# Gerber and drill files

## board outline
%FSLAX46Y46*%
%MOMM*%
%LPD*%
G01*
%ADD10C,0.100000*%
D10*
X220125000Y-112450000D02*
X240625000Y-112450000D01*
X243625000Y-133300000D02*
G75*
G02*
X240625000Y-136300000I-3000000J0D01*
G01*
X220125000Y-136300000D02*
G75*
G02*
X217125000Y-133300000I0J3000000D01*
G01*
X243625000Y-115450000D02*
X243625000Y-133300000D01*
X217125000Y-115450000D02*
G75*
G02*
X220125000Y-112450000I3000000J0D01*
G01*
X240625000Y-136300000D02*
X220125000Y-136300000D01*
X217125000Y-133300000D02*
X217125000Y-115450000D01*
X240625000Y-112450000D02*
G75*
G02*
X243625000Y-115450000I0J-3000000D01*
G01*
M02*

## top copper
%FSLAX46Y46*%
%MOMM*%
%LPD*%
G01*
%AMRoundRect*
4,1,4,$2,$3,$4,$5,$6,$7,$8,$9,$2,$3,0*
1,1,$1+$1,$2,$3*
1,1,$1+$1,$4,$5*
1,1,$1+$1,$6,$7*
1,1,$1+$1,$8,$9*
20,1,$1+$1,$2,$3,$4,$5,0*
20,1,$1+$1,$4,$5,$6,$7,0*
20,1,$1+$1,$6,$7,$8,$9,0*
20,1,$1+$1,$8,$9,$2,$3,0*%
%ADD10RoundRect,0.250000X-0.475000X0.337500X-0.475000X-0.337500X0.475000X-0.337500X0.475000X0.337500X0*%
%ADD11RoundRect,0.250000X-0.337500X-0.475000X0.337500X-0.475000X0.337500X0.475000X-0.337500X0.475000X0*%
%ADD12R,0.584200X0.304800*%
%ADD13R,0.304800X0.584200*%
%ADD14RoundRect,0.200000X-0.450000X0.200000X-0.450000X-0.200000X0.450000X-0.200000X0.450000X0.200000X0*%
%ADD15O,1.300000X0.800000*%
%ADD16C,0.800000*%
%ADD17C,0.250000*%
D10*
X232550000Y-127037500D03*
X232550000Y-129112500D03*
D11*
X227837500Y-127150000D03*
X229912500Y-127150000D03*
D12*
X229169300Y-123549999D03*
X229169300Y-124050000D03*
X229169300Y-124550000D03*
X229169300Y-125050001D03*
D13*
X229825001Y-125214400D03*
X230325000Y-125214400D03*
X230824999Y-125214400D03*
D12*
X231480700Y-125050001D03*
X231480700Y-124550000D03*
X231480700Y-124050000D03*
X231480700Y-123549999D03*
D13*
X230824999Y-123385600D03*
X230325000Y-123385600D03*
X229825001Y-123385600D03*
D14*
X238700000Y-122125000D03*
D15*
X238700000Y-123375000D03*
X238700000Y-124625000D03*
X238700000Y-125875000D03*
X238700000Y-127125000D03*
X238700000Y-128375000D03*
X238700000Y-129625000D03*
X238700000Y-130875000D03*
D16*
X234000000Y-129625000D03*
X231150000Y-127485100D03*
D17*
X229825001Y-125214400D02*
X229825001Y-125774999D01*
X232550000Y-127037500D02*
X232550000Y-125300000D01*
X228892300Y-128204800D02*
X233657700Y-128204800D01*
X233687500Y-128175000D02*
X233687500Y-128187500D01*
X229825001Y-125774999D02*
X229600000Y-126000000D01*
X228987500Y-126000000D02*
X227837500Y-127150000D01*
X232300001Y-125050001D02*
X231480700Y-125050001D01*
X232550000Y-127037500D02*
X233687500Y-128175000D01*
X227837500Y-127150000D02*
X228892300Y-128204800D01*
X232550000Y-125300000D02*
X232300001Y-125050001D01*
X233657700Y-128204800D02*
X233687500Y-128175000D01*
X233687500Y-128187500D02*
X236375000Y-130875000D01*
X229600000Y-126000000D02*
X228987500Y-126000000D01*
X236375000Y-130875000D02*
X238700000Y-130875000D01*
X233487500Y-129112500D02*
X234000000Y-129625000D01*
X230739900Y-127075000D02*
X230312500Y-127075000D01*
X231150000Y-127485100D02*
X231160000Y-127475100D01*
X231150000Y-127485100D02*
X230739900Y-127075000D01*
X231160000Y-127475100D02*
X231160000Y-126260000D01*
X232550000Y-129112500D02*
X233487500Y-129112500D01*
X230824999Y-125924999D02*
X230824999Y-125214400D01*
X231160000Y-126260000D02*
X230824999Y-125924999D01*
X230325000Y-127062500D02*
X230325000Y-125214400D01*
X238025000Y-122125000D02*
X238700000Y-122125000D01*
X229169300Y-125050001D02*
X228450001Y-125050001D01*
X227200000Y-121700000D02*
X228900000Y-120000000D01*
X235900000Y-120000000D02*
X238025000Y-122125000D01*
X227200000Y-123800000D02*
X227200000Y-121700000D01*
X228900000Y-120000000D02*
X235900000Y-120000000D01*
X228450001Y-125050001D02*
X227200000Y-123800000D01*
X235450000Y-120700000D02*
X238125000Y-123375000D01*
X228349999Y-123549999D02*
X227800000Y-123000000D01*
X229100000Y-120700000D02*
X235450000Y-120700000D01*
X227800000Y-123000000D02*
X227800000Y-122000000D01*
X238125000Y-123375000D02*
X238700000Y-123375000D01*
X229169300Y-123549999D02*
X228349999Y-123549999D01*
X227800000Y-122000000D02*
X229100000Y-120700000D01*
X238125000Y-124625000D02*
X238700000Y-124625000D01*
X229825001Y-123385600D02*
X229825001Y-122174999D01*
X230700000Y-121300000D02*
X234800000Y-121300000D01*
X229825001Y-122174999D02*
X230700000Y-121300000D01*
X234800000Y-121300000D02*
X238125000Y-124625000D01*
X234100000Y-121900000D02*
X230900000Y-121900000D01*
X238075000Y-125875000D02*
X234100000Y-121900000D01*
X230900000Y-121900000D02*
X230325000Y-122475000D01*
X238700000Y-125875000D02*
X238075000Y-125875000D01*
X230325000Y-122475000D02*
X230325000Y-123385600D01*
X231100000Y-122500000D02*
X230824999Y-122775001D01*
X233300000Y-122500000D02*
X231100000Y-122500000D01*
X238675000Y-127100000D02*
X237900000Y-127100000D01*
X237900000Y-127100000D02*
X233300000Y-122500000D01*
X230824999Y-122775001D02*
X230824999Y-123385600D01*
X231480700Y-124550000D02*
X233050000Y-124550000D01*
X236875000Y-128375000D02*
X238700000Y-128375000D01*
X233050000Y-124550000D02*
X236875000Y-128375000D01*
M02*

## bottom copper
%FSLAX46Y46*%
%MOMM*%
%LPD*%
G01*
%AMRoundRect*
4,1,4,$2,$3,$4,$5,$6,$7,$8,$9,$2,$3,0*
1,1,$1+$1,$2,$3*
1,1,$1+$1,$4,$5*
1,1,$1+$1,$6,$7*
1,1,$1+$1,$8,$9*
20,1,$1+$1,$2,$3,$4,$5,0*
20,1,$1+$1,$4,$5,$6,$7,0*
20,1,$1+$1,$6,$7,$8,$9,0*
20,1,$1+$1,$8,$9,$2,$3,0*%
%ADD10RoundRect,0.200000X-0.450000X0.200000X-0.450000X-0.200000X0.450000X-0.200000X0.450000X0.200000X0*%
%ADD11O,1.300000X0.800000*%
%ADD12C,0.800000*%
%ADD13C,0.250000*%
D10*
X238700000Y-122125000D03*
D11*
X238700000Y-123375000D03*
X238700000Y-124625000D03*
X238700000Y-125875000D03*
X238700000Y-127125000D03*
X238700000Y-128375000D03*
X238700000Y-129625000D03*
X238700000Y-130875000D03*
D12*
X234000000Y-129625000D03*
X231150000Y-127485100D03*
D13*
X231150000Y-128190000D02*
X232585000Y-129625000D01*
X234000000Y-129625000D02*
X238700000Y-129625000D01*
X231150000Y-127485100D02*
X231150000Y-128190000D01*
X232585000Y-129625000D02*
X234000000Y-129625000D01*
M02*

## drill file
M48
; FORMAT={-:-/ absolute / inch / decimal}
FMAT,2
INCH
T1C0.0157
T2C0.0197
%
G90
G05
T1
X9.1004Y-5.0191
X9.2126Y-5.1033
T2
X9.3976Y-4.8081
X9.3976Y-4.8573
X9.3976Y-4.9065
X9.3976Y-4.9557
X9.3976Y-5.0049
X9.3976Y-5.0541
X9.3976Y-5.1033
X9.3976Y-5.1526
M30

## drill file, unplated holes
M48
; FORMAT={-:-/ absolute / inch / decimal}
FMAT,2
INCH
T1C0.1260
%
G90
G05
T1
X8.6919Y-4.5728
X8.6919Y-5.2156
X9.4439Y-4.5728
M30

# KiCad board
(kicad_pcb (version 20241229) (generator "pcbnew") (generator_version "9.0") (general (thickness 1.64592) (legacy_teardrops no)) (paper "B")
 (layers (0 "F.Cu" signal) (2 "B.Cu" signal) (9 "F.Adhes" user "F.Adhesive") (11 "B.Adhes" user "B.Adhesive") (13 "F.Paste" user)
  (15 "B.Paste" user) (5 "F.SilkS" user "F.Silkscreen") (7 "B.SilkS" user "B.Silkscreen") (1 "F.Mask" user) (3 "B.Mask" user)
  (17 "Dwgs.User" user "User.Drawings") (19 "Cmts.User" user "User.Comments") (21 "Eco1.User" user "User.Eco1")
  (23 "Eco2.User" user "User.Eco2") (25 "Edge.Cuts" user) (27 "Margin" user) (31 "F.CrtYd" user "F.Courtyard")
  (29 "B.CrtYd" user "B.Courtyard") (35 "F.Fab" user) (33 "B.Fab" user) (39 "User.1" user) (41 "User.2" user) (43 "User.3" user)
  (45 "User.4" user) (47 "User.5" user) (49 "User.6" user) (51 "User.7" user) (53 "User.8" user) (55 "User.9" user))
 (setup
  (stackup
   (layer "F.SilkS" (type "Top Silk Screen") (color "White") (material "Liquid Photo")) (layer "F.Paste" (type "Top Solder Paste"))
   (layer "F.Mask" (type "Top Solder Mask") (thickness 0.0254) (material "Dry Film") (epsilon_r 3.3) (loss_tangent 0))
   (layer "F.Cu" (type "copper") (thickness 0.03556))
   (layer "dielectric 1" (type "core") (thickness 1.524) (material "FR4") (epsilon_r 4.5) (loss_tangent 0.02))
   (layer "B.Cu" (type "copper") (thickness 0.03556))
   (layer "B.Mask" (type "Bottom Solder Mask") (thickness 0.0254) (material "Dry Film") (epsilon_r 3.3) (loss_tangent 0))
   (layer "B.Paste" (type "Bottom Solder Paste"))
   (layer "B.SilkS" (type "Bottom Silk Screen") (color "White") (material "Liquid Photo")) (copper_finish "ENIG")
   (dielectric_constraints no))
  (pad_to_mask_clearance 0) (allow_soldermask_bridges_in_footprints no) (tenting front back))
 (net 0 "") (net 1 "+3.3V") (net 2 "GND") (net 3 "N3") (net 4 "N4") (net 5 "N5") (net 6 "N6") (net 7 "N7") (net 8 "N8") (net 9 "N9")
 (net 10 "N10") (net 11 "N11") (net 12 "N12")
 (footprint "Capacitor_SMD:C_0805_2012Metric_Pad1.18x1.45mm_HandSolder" (layer "F.Cu") (at 232.55 128.075 -90)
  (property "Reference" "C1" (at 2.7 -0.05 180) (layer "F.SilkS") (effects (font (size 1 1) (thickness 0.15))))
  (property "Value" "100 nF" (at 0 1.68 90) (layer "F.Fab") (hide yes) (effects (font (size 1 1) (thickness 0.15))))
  (pad "1" smd roundrect (at -1.0375 0 270) (size 1.175 1.45) (layers "F.Cu" "F.Mask" "F.Paste") (roundrect_rratio 0.2127659574)
   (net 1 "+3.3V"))
  (pad "2" smd roundrect (at 1.0375 0 270) (size 1.175 1.45) (layers "F.Cu" "F.Mask" "F.Paste") (roundrect_rratio 0.2127659574)
   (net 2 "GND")))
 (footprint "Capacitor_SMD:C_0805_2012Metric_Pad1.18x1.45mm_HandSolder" (layer "F.Cu") (at 228.875 127.15)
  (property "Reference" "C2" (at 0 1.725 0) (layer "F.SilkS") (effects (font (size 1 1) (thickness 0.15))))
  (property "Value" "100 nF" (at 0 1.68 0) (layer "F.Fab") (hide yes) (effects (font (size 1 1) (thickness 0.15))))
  (pad "1" smd roundrect (at -1.0375 0) (size 1.175 1.45) (layers "F.Cu" "F.Mask" "F.Paste") (roundrect_rratio 0.2127659574) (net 1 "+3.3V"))
  (pad "2" smd roundrect (at 1.0375 0) (size 1.175 1.45) (layers "F.Cu" "F.Mask" "F.Paste") (roundrect_rratio 0.2127659574) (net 2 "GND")))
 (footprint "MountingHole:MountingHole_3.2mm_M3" (layer "F.Cu") (at 220.775 132.475)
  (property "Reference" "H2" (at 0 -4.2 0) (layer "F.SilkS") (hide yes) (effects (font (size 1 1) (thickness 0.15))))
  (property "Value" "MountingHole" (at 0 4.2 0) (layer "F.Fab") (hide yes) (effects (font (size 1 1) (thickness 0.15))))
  (pad "" np_thru_hole circle (at 0 0) (size 3.2 3.2) (drill 3.2) (layers "*.Cu" "*.Mask")))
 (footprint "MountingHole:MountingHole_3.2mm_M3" (layer "F.Cu") (at 239.875 116.15)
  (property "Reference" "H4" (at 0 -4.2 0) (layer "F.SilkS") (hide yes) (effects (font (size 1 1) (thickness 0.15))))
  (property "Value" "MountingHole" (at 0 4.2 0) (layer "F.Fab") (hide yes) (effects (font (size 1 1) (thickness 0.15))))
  (pad "" np_thru_hole circle (at 0 0) (size 3.2 3.2) (drill 3.2) (layers "*.Cu" "*.Mask")))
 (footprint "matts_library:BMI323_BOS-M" (layer "F.Cu") (at 230.325 124.3)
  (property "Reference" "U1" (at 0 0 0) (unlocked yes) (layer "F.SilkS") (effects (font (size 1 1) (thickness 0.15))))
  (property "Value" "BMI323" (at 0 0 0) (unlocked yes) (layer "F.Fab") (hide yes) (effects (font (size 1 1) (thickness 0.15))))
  (pad "1" smd rect (at -1.1557 -0.750001 90) (size 0.3048 0.5842) (layers "F.Cu" "F.Mask" "F.Paste") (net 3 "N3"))
  (pad "2" smd rect (at -1.1557 -0.25 90) (size 0.3048 0.5842) (layers "F.Cu" "F.Mask" "F.Paste") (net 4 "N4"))
  (pad "3" smd rect (at -1.1557 0.25 90) (size 0.3048 0.5842) (layers "F.Cu" "F.Mask" "F.Paste") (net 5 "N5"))
  (pad "4" smd rect (at -1.1557 0.750001 90) (size 0.3048 0.5842) (layers "F.Cu" "F.Mask" "F.Paste") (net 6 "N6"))
  (pad "5" smd rect (at -0.499999 0.9144) (size 0.3048 0.5842) (layers "F.Cu" "F.Mask" "F.Paste") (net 1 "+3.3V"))
  (pad "6" smd rect (at 0 0.9144) (size 0.3048 0.5842) (layers "F.Cu" "F.Mask" "F.Paste") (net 2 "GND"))
  (pad "7" smd rect (at 0.499999 0.9144) (size 0.3048 0.5842) (layers "F.Cu" "F.Mask" "F.Paste") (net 2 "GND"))
  (pad "8" smd rect (at 1.1557 0.750001 90) (size 0.3048 0.5842) (layers "F.Cu" "F.Mask" "F.Paste") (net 1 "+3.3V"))
  (pad "9" smd rect (at 1.1557 0.25 90) (size 0.3048 0.5842) (layers "F.Cu" "F.Mask" "F.Paste") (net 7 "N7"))
  (pad "10" smd rect (at 1.1557 -0.25 90) (size 0.3048 0.5842) (layers "F.Cu" "F.Mask" "F.Paste") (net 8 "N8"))
  (pad "11" smd rect (at 1.1557 -0.750001 90) (size 0.3048 0.5842) (layers "F.Cu" "F.Mask" "F.Paste") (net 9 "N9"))
  (pad "12" smd rect (at 0.499999 -0.9144) (size 0.3048 0.5842) (layers "F.Cu" "F.Mask" "F.Paste") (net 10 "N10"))
  (pad "13" smd rect (at 0 -0.9144) (size 0.3048 0.5842) (layers "F.Cu" "F.Mask" "F.Paste") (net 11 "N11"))
  (pad "14" smd rect (at -0.499999 -0.9144) (size 0.3048 0.5842) (layers "F.Cu" "F.Mask" "F.Paste") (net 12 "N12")))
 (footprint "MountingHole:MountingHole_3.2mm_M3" (layer "F.Cu") (at 220.775 116.15)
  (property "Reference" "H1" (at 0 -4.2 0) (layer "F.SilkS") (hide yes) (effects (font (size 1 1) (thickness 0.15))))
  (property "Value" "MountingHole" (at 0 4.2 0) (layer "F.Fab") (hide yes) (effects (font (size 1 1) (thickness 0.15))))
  (pad "" np_thru_hole circle (at 0 0) (size 3.2 3.2) (drill 3.2) (layers "*.Cu" "*.Mask")))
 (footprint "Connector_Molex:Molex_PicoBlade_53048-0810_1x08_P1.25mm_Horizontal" (layer "B.Cu") (at 238.7 122.125 -90)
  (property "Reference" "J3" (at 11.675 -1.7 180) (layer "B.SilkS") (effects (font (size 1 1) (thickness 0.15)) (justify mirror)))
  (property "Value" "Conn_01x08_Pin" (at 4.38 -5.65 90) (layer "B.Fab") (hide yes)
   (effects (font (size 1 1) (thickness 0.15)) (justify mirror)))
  (pad "1" thru_hole roundrect (at 0 0 270) (size 0.8 1.3) (drill 0.5) (layers "*.Cu" "*.Mask") (remove_unused_layers no)
   (roundrect_rratio 0.25) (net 6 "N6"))
  (pad "2" thru_hole oval (at 1.25 0 270) (size 0.8 1.3) (drill 0.5) (layers "*.Cu" "*.Mask") (remove_unused_layers no) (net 3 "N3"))
  (pad "3" thru_hole oval (at 2.5 0 270) (size 0.8 1.3) (drill 0.5) (layers "*.Cu" "*.Mask") (remove_unused_layers no) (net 12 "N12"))
  (pad "4" thru_hole oval (at 3.75 0 270) (size 0.8 1.3) (drill 0.5) (layers "*.Cu" "*.Mask") (remove_unused_layers no) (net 11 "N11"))
  (pad "5" thru_hole oval (at 5 0 270) (size 0.8 1.3) (drill 0.5) (layers "*.Cu" "*.Mask") (remove_unused_layers no) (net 10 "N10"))
  (pad "6" thru_hole oval (at 6.25 0 270) (size 0.8 1.3) (drill 0.5) (layers "*.Cu" "*.Mask") (remove_unused_layers no) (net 7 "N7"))
  (pad "7" thru_hole oval (at 7.5 0 270) (size 0.8 1.3) (drill 0.5) (layers "*.Cu" "*.Mask") (remove_unused_layers no) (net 2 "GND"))
  (pad "8" thru_hole oval (at 8.75 0 270) (size 0.8 1.3) (drill 0.5) (layers "*.Cu" "*.Mask") (remove_unused_layers no) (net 1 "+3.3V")))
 (gr_line (start 220.125 112.45) (end 240.625 112.45) (stroke (width 0.1) (type default)) (layer "Edge.Cuts"))
 (gr_arc (start 243.625 133.3) (mid 242.74632 135.42132) (end 240.625 136.3) (stroke (width 0.1) (type default)) (layer "Edge.Cuts"))
 (gr_arc (start 220.125 136.3) (mid 218.00368 135.42132) (end 217.125 133.3) (stroke (width 0.1) (type default)) (layer "Edge.Cuts"))
 (gr_line (start 243.625 115.45) (end 243.625 133.3) (stroke (width 0.1) (type default)) (layer "Edge.Cuts"))
 (gr_arc (start 217.125 115.45) (mid 218.00368 113.32868) (end 220.125 112.45) (stroke (width 0.1) (type default)) (layer "Edge.Cuts"))
 (gr_line (start 240.625 136.3) (end 220.125 136.3) (stroke (width 0.1) (type default)) (layer "Edge.Cuts"))
 (gr_line (start 217.125 133.3) (end 217.125 115.45) (stroke (width 0.1) (type default)) (layer "Edge.Cuts"))
 (gr_arc (start 240.625 112.45) (mid 242.74632 113.32868) (end 243.625 115.45) (stroke (width 0.1) (type default)) (layer "Edge.Cuts"))
 (segment (start 229.825001 125.2144) (end 229.825001 125.774999) (width 0.25) (layer "F.Cu") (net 1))
 (segment (start 232.55 127.0375) (end 232.55 125.3) (width 0.25) (layer "F.Cu") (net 1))
 (segment (start 228.8923 128.2048) (end 233.6577 128.2048) (width 0.25) (layer "F.Cu") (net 1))
 (segment (start 233.6875 128.175) (end 233.6875 128.1875) (width 0.25) (layer "F.Cu") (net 1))
 (segment (start 229.825001 125.774999) (end 229.6 126) (width 0.25) (layer "F.Cu") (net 1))
 (segment (start 228.9875 126) (end 227.8375 127.15) (width 0.25) (layer "F.Cu") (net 1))
 (segment (start 232.300001 125.050001) (end 231.4807 125.050001) (width 0.25) (layer "F.Cu") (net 1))
 (segment (start 232.55 127.0375) (end 233.6875 128.175) (width 0.25) (layer "F.Cu") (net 1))
 (segment (start 227.8375 127.15) (end 228.8923 128.2048) (width 0.25) (layer "F.Cu") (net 1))
 (segment (start 232.55 125.3) (end 232.300001 125.050001) (width 0.25) (layer "F.Cu") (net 1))
 (segment (start 233.6577 128.2048) (end 233.6875 128.175) (width 0.25) (layer "F.Cu") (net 1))
 (segment (start 233.6875 128.1875) (end 236.375 130.875) (width 0.25) (layer "F.Cu") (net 1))
 (segment (start 229.6 126) (end 228.9875 126) (width 0.25) (layer "F.Cu") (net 1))
 (segment (start 236.375 130.875) (end 238.7 130.875) (width 0.25) (layer "F.Cu") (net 1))
 (segment (start 233.4875 129.1125) (end 234 129.625) (width 0.25) (layer "F.Cu") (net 2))
 (segment (start 230.7399 127.075) (end 230.3125 127.075) (width 0.25) (layer "F.Cu") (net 2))
 (segment (start 231.15 127.4851) (end 231.16 127.4751) (width 0.25) (layer "F.Cu") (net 2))
 (segment (start 231.15 127.4851) (end 230.7399 127.075) (width 0.25) (layer "F.Cu") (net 2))
 (segment (start 231.16 127.4751) (end 231.16 126.26) (width 0.25) (layer "F.Cu") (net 2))
 (segment (start 232.55 129.1125) (end 233.4875 129.1125) (width 0.25) (layer "F.Cu") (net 2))
 (segment (start 230.824999 125.924999) (end 230.824999 125.2144) (width 0.25) (layer "F.Cu") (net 2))
 (segment (start 231.16 126.26) (end 230.824999 125.924999) (width 0.25) (layer "F.Cu") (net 2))
 (segment (start 230.325 127.0625) (end 230.325 125.2144) (width 0.25) (layer "F.Cu") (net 2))
 (via (at 234 129.625) (size 0.8) (drill 0.4) (layers "F.Cu" "B.Cu") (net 2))
 (via (at 231.15 127.4851) (size 0.8) (drill 0.4) (layers "F.Cu" "B.Cu") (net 2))
 (segment (start 231.15 128.19) (end 232.585 129.625) (width 0.25) (layer "B.Cu") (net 2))
 (segment (start 234 129.625) (end 238.7 129.625) (width 0.25) (layer "B.Cu") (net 2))
 (segment (start 231.15 127.4851) (end 231.15 128.19) (width 0.25) (layer "B.Cu") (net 2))
 (segment (start 232.585 129.625) (end 234 129.625) (width 0.25) (layer "B.Cu") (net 2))
 (segment (start 238.025 122.125) (end 238.7 122.125) (width 0.25) (layer "F.Cu") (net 6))
 (segment (start 229.1693 125.050001) (end 228.450001 125.050001) (width 0.25) (layer "F.Cu") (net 6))
 (segment (start 227.2 121.7) (end 228.9 120) (width 0.25) (layer "F.Cu") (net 6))
 (segment (start 235.9 120) (end 238.025 122.125) (width 0.25) (layer "F.Cu") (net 6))
 (segment (start 227.2 123.8) (end 227.2 121.7) (width 0.25) (layer "F.Cu") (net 6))
 (segment (start 228.9 120) (end 235.9 120) (width 0.25) (layer "F.Cu") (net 6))
 (segment (start 228.450001 125.050001) (end 227.2 123.8) (width 0.25) (layer "F.Cu") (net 6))
 (segment (start 235.45 120.7) (end 238.125 123.375) (width 0.25) (layer "F.Cu") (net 3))
 (segment (start 228.349999 123.549999) (end 227.8 123) (width 0.25) (layer "F.Cu") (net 3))
 (segment (start 229.1 120.7) (end 235.45 120.7) (width 0.25) (layer "F.Cu") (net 3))
 (segment (start 227.8 123) (end 227.8 122) (width 0.25) (layer "F.Cu") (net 3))
 (segment (start 238.125 123.375) (end 238.7 123.375) (width 0.25) (layer "F.Cu") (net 3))
 (segment (start 229.1693 123.549999) (end 228.349999 123.549999) (width 0.25) (layer "F.Cu") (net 3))
 (segment (start 227.8 122) (end 229.1 120.7) (width 0.25) (layer "F.Cu") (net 3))
 (segment (start 238.125 124.625) (end 238.7 124.625) (width 0.25) (layer "F.Cu") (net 12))
 (segment (start 229.825001 123.3856) (end 229.825001 122.174999) (width 0.25) (layer "F.Cu") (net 12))
 (segment (start 230.7 121.3) (end 234.8 121.3) (width 0.25) (layer "F.Cu") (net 12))
 (segment (start 229.825001 122.174999) (end 230.7 121.3) (width 0.25) (layer "F.Cu") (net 12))
 (segment (start 234.8 121.3) (end 238.125 124.625) (width 0.25) (layer "F.Cu") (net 12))
 (segment (start 234.1 121.9) (end 230.9 121.9) (width 0.25) (layer "F.Cu") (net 11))
 (segment (start 238.075 125.875) (end 234.1 121.9) (width 0.25) (layer "F.Cu") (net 11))
 (segment (start 230.9 121.9) (end 230.325 122.475) (width 0.25) (layer "F.Cu") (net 11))
 (segment (start 238.7 125.875) (end 238.075 125.875) (width 0.25) (layer "F.Cu") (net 11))
 (segment (start 230.325 122.475) (end 230.325 123.3856) (width 0.25) (layer "F.Cu") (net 11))
 (segment (start 231.1 122.5) (end 230.824999 122.775001) (width 0.25) (layer "F.Cu") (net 10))
 (segment (start 233.3 122.5) (end 231.1 122.5) (width 0.25) (layer "F.Cu") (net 10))
 (segment (start 238.675 127.1) (end 237.9 127.1) (width 0.25) (layer "F.Cu") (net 10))
 (segment (start 237.9 127.1) (end 233.3 122.5) (width 0.25) (layer "F.Cu") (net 10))
 (segment (start 230.824999 122.775001) (end 230.824999 123.3856) (width 0.25) (layer "F.Cu") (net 10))
 (segment (start 231.4807 124.55) (end 233.05 124.55) (width 0.25) (layer "F.Cu") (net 7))
 (segment (start 236.875 128.375) (end 238.7 128.375) (width 0.25) (layer "F.Cu") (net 7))
 (segment (start 233.05 124.55) (end 236.875 128.375) (width 0.25) (layer "F.Cu") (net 7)))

